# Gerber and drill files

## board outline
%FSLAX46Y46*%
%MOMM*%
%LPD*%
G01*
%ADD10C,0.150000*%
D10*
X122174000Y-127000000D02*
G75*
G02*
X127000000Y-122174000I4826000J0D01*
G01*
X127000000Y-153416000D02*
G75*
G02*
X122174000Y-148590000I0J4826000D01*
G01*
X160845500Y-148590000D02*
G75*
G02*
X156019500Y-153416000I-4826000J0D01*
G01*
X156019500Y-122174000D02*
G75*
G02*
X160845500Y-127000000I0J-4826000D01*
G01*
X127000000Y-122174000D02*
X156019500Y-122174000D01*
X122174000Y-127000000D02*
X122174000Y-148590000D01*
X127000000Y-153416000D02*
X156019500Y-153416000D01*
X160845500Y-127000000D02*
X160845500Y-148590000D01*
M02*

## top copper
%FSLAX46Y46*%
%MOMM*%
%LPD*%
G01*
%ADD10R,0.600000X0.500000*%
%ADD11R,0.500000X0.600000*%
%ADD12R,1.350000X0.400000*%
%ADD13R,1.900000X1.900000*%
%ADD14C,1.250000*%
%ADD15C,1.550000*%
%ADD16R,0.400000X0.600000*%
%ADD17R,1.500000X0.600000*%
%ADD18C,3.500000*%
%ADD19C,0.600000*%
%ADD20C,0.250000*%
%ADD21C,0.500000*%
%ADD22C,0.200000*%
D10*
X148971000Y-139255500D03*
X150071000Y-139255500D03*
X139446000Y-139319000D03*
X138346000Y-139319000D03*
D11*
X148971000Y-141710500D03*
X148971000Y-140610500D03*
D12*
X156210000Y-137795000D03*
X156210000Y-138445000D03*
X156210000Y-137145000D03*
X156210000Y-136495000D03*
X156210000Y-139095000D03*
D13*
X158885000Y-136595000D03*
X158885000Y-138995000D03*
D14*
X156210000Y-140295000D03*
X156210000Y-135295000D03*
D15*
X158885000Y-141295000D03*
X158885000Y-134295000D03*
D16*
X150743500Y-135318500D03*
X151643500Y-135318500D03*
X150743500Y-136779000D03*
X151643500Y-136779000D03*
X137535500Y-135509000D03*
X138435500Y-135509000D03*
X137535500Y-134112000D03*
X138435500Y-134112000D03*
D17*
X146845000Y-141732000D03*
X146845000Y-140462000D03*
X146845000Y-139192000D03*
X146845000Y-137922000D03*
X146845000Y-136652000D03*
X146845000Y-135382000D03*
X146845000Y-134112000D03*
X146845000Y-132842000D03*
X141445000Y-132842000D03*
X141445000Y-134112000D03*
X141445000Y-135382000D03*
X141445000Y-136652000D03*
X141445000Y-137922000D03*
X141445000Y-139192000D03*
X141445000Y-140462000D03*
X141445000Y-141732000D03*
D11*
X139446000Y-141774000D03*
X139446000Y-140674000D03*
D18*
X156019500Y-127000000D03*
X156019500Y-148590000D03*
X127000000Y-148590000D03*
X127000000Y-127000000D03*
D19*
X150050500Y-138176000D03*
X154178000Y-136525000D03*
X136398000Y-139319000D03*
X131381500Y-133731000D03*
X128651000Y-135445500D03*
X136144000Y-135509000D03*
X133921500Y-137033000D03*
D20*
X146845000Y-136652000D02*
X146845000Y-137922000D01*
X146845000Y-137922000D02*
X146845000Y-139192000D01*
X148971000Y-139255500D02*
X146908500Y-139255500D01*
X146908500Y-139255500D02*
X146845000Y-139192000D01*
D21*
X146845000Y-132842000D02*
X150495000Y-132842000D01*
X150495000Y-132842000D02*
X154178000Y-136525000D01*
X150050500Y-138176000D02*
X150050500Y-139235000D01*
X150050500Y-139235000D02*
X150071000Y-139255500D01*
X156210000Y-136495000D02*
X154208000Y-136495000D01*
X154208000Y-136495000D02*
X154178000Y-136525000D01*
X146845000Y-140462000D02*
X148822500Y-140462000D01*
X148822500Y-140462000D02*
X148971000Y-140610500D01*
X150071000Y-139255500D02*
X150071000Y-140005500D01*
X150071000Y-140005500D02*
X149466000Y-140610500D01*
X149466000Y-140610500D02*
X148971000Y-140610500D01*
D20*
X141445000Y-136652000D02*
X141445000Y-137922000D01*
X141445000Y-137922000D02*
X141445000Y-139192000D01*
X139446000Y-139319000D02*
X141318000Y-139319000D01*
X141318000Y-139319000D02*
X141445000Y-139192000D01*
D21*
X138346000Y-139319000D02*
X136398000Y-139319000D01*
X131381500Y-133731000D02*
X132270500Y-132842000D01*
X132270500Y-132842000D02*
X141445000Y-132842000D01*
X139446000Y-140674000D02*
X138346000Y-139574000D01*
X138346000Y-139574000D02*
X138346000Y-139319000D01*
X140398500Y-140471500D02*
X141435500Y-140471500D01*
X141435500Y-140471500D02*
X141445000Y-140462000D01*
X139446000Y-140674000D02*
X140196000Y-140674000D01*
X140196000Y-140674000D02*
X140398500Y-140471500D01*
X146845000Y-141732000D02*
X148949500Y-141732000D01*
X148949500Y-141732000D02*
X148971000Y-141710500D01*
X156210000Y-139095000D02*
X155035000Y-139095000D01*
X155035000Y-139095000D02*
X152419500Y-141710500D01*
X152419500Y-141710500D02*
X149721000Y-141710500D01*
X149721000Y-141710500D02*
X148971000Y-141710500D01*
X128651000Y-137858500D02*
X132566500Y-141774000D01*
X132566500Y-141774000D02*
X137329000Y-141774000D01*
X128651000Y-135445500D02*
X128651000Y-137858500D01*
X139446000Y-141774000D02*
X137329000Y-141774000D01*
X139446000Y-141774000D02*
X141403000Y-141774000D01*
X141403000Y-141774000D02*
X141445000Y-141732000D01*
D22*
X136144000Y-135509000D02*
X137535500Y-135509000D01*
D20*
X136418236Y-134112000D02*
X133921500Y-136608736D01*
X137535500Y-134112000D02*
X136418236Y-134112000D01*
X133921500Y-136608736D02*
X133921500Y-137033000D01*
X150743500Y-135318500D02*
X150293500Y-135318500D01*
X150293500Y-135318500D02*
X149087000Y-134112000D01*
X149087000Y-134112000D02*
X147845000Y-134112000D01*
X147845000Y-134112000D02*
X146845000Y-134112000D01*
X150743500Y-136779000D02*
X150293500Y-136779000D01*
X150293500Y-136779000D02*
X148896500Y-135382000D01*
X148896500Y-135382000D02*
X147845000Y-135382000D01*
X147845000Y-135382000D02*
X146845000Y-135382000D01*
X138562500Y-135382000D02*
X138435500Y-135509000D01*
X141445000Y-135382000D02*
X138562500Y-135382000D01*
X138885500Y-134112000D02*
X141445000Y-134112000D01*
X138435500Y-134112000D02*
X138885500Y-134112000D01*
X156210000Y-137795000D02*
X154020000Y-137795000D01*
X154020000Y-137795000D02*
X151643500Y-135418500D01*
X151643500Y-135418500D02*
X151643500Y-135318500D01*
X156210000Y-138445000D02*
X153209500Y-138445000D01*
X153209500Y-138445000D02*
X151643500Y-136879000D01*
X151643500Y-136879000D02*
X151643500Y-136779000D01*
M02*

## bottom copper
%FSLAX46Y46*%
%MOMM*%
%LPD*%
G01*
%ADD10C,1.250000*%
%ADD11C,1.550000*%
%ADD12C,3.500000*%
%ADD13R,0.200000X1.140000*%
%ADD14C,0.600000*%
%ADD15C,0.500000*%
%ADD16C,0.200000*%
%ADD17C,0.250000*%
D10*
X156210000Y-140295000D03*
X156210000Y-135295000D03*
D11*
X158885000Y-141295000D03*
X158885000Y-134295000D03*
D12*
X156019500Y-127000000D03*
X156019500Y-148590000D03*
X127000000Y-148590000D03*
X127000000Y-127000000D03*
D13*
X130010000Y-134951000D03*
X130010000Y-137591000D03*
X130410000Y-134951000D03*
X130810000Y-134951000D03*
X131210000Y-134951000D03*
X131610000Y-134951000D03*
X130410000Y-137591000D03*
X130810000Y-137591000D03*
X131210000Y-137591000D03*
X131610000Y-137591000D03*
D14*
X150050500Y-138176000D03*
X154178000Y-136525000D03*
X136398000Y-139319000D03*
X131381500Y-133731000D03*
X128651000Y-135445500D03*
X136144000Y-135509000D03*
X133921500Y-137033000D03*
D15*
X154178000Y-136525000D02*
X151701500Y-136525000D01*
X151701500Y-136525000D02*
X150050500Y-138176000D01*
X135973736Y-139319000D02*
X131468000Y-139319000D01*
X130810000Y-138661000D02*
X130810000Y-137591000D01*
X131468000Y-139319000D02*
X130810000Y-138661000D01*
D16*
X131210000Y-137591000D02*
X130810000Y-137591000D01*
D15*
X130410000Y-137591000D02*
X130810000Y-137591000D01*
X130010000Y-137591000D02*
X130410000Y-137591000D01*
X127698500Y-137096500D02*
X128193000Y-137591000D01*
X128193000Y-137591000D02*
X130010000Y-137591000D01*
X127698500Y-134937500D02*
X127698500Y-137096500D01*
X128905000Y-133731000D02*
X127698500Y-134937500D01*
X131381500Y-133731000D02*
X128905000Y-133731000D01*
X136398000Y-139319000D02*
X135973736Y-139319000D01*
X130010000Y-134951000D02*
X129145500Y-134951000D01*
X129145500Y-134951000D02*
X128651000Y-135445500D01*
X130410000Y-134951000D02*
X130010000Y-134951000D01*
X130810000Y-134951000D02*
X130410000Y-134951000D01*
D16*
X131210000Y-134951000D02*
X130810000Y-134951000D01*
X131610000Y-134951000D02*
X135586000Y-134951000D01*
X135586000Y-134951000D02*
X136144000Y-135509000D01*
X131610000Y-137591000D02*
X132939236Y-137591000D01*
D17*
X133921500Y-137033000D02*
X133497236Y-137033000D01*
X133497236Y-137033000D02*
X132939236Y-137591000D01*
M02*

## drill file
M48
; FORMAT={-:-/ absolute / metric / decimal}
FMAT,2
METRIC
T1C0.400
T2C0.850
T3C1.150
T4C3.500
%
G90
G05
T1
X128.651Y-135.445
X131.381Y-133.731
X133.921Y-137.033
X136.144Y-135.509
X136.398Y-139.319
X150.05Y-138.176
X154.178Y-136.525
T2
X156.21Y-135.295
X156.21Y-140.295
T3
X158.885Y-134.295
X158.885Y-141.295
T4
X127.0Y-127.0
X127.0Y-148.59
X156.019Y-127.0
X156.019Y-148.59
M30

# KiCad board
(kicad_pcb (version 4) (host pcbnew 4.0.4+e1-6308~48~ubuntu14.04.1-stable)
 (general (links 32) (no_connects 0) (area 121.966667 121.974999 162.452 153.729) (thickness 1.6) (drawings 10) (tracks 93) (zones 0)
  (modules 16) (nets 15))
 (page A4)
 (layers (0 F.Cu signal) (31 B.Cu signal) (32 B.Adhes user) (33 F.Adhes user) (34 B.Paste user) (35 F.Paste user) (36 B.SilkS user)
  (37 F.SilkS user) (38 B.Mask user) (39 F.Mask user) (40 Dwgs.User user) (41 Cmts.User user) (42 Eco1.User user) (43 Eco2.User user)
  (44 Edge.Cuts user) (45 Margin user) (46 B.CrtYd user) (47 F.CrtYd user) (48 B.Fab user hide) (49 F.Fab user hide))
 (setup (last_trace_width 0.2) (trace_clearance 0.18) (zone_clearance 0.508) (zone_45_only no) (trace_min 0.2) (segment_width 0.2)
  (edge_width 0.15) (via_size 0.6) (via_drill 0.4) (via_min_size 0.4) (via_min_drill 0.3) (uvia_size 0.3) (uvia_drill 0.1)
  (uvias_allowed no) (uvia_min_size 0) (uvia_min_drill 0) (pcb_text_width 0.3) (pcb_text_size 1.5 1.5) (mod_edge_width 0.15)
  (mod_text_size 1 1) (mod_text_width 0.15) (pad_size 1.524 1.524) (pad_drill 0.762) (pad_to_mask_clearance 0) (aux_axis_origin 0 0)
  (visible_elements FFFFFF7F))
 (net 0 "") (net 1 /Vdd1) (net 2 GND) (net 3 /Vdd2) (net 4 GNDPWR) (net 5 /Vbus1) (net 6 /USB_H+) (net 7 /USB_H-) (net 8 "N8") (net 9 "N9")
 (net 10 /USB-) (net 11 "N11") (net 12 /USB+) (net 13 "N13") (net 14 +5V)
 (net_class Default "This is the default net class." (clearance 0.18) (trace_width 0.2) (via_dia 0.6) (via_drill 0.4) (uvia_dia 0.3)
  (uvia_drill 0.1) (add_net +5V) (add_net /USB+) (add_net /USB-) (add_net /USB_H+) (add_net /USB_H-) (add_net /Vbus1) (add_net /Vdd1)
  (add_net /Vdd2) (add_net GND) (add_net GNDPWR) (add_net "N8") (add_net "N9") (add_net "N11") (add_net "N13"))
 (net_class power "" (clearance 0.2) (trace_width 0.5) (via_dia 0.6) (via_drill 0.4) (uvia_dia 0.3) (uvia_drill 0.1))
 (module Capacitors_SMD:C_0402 (layer F.Cu) (at 149.521 139.2555)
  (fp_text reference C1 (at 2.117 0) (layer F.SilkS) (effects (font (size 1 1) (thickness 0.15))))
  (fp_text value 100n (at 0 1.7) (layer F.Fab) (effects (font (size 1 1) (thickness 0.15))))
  (pad 1 smd rect (at -0.55 0) (size 0.6 0.5) (layers F.Cu F.Paste F.Mask) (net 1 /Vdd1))
  (pad 2 smd rect (at 0.55 0) (size 0.6 0.5) (layers F.Cu F.Paste F.Mask) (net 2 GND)))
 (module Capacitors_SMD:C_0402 (layer F.Cu) (at 138.896 139.319 180)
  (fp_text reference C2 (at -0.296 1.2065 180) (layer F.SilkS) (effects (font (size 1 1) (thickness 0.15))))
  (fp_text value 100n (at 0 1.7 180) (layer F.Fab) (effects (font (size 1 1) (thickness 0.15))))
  (pad 1 smd rect (at -0.55 0 180) (size 0.6 0.5) (layers F.Cu F.Paste F.Mask) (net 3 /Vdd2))
  (pad 2 smd rect (at 0.55 0 180) (size 0.6 0.5) (layers F.Cu F.Paste F.Mask) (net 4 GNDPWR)))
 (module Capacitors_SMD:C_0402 (layer F.Cu) (at 148.971 141.1605 90)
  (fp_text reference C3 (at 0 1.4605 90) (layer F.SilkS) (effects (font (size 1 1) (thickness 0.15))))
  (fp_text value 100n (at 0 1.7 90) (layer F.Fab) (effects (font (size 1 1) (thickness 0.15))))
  (pad 1 smd rect (at -0.55 0 90) (size 0.6 0.5) (layers F.Cu F.Paste F.Mask) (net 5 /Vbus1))
  (pad 2 smd rect (at 0.55 0 90) (size 0.6 0.5) (layers F.Cu F.Paste F.Mask) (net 2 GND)))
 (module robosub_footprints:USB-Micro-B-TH (layer F.Cu) (at 155.535 137.795 90)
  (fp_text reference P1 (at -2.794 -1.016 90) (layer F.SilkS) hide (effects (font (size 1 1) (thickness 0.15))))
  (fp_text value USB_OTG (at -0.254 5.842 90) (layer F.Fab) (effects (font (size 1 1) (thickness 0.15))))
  (pad 3 smd rect (at 0 0.675 90) (size 0.4 1.35) (layers F.Cu F.Paste F.Mask) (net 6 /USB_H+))
  (pad 2 smd rect (at -0.65 0.675 90) (size 0.4 1.35) (layers F.Cu F.Paste F.Mask) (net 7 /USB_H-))
  (pad 4 smd rect (at 0.65 0.675 90) (size 0.4 1.35) (layers F.Cu F.Paste F.Mask))
  (pad 5 smd rect (at 1.3 0.675 90) (size 0.4 1.35) (layers F.Cu F.Paste F.Mask) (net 2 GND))
  (pad 1 smd rect (at -1.3 0.675 90) (size 0.4 1.35) (layers F.Cu F.Paste F.Mask) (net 5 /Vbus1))
  (pad "" smd rect (at 1.2 3.35 90) (size 1.9 1.9) (layers F.Cu F.Paste F.Mask))
  (pad "" smd rect (at -1.2 3.35 90) (size 1.9 1.9) (layers F.Cu F.Paste F.Mask))
  (pad "" thru_hole circle (at -2.5 0.675 90) (size 1.25 1.25) (drill 0.85) (layers *.Cu *.Mask F.SilkS))
  (pad "" thru_hole circle (at 2.5 0.675 90) (size 1.25 1.25) (drill 0.85) (layers *.Cu *.Mask F.SilkS))
  (pad "" thru_hole circle (at -3.5 3.35 90) (size 1.55 1.55) (drill 1.15) (layers *.Cu *.Mask F.SilkS))
  (pad "" thru_hole circle (at 3.5 3.35 90) (size 1.55 1.55) (drill 1.15) (layers *.Cu *.Mask F.SilkS)))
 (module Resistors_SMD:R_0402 (layer F.Cu) (at 151.1935 135.3185)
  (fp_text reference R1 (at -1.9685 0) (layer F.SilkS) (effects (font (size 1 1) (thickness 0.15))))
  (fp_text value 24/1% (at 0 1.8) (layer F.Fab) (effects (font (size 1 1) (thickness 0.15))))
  (pad 1 smd rect (at -0.45 0) (size 0.4 0.6) (layers F.Cu F.Paste F.Mask) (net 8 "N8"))
  (pad 2 smd rect (at 0.45 0) (size 0.4 0.6) (layers F.Cu F.Paste F.Mask) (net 6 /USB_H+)))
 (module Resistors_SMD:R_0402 (layer F.Cu) (at 151.1935 136.779)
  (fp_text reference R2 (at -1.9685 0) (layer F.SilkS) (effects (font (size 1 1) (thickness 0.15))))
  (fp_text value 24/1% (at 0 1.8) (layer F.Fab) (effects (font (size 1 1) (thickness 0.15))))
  (pad 1 smd rect (at -0.45 0) (size 0.4 0.6) (layers F.Cu F.Paste F.Mask) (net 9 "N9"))
  (pad 2 smd rect (at 0.45 0) (size 0.4 0.6) (layers F.Cu F.Paste F.Mask) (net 7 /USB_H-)))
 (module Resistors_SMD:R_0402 (layer F.Cu) (at 137.9855 135.509)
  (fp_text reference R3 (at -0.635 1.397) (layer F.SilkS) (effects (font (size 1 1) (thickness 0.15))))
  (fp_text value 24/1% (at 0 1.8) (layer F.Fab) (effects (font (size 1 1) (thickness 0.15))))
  (pad 1 smd rect (at -0.45 0) (size 0.4 0.6) (layers F.Cu F.Paste F.Mask) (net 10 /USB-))
  (pad 2 smd rect (at 0.45 0) (size 0.4 0.6) (layers F.Cu F.Paste F.Mask) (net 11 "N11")))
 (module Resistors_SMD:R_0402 (layer F.Cu) (at 137.9855 134.112)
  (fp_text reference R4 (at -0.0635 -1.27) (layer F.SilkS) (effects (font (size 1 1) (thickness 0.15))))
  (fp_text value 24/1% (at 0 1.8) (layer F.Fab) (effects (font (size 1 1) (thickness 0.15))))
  (pad 1 smd rect (at -0.45 0) (size 0.4 0.6) (layers F.Cu F.Paste F.Mask) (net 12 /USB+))
  (pad 2 smd rect (at 0.45 0) (size 0.4 0.6) (layers F.Cu F.Paste F.Mask) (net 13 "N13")))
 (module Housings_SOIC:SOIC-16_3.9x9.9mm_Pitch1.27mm (layer F.Cu) (at 144.145 137.287 180)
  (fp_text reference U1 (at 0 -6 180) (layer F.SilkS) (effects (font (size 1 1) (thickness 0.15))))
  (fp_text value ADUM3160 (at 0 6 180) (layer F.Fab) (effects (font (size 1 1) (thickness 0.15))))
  (pad 1 smd rect (at -2.7 -4.445 180) (size 1.5 0.6) (layers F.Cu F.Paste F.Mask) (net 5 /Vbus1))
  (pad 2 smd rect (at -2.7 -3.175 180) (size 1.5 0.6) (layers F.Cu F.Paste F.Mask) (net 2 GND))
  (pad 3 smd rect (at -2.7 -1.905 180) (size 1.5 0.6) (layers F.Cu F.Paste F.Mask) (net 1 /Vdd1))
  (pad 4 smd rect (at -2.7 -0.635 180) (size 1.5 0.6) (layers F.Cu F.Paste F.Mask) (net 1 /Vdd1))
  (pad 5 smd rect (at -2.7 0.635 180) (size 1.5 0.6) (layers F.Cu F.Paste F.Mask) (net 1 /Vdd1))
  (pad 6 smd rect (at -2.7 1.905 180) (size 1.5 0.6) (layers F.Cu F.Paste F.Mask) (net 9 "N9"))
  (pad 7 smd rect (at -2.7 3.175 180) (size 1.5 0.6) (layers F.Cu F.Paste F.Mask) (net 8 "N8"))
  (pad 8 smd rect (at -2.7 4.445 180) (size 1.5 0.6) (layers F.Cu F.Paste F.Mask) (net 2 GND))
  (pad 9 smd rect (at 2.7 4.445 180) (size 1.5 0.6) (layers F.Cu F.Paste F.Mask) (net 4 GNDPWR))
  (pad 10 smd rect (at 2.7 3.175 180) (size 1.5 0.6) (layers F.Cu F.Paste F.Mask) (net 13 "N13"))
  (pad 11 smd rect (at 2.7 1.905 180) (size 1.5 0.6) (layers F.Cu F.Paste F.Mask) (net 11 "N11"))
  (pad 12 smd rect (at 2.7 0.635 180) (size 1.5 0.6) (layers F.Cu F.Paste F.Mask) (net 3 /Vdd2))
  (pad 13 smd rect (at 2.7 -0.635 180) (size 1.5 0.6) (layers F.Cu F.Paste F.Mask) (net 3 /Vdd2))
  (pad 14 smd rect (at 2.7 -1.905 180) (size 1.5 0.6) (layers F.Cu F.Paste F.Mask) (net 3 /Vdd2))
  (pad 15 smd rect (at 2.7 -3.175 180) (size 1.5 0.6) (layers F.Cu F.Paste F.Mask) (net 4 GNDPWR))
  (pad 16 smd rect (at 2.7 -4.445 180) (size 1.5 0.6) (layers F.Cu F.Paste F.Mask) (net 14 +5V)))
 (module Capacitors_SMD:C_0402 (layer F.Cu) (at 139.446 141.224 90)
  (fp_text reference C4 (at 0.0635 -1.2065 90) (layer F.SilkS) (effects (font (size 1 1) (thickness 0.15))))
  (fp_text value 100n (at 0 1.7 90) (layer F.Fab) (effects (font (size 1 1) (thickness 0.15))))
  (pad 1 smd rect (at -0.55 0 90) (size 0.6 0.5) (layers F.Cu F.Paste F.Mask) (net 14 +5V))
  (pad 2 smd rect (at 0.55 0 90) (size 0.6 0.5) (layers F.Cu F.Paste F.Mask) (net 4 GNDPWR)))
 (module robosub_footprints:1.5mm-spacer (layer F.Cu) (at 156.0195 127)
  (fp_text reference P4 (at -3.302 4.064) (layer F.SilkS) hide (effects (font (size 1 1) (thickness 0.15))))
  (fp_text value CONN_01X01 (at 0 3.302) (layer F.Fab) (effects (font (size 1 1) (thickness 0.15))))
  (pad "" thru_hole circle (at 0 0) (size 3.5 3.5) (drill 3.5) (layers *.Cu *.Mask F.SilkS)))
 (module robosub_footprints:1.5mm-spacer (layer F.Cu) (at 156.0195 148.59)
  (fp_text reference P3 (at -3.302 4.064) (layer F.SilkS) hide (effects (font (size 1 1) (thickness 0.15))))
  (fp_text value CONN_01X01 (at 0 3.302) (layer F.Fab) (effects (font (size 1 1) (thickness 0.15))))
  (pad "" thru_hole circle (at 0 0) (size 3.5 3.5) (drill 3.5) (layers *.Cu *.Mask F.SilkS)))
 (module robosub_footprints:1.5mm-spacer (layer F.Cu) (at 127 148.59)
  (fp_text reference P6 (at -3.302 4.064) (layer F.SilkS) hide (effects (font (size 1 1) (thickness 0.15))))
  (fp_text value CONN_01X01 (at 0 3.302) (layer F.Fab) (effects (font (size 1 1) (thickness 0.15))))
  (pad "" thru_hole circle (at 0 0) (size 3.5 3.5) (drill 3.5) (layers *.Cu *.Mask F.SilkS)))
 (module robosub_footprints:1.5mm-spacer (layer F.Cu) (at 127 127)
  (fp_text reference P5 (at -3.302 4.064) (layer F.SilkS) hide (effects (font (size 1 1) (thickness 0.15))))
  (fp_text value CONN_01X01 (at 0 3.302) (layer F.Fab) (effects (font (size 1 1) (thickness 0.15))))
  (pad "" thru_hole circle (at 0 0) (size 3.5 3.5) (drill 3.5) (layers *.Cu *.Mask F.SilkS)))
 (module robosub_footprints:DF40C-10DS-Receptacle (layer B.Cu) (at 130.81 136.271)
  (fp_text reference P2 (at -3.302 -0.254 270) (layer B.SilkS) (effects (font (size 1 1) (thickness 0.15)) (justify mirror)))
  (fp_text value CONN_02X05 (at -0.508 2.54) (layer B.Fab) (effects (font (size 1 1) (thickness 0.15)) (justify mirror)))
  (pad 1 smd rect (at -0.8 -1.32 270) (size 1.14 0.2) (layers B.Cu B.Paste B.Mask) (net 14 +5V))
  (pad 2 smd rect (at -0.8 1.32 270) (size 1.14 0.2) (layers B.Cu B.Paste B.Mask) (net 4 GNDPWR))
  (pad 3 smd rect (at -0.4 -1.32 270) (size 1.14 0.2) (layers B.Cu B.Paste B.Mask) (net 14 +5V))
  (pad 5 smd rect (at 0 -1.32 270) (size 1.14 0.2) (layers B.Cu B.Paste B.Mask) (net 14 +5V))
  (pad 7 smd rect (at 0.4 -1.32 270) (size 1.14 0.2) (layers B.Cu B.Paste B.Mask) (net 14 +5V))
  (pad 9 smd rect (at 0.8 -1.32 270) (size 1.14 0.2) (layers B.Cu B.Paste B.Mask) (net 10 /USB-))
  (pad 4 smd rect (at -0.4 1.32 270) (size 1.14 0.2) (layers B.Cu B.Paste B.Mask) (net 4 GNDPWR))
  (pad 6 smd rect (at 0 1.32 270) (size 1.14 0.2) (layers B.Cu B.Paste B.Mask) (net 4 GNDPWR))
  (pad 8 smd rect (at 0.4 1.32 270) (size 1.14 0.2) (layers B.Cu B.Paste B.Mask) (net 4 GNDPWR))
  (pad 10 smd rect (at 0.8 1.32 270) (size 1.14 0.2) (layers B.Cu B.Paste B.Mask) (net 12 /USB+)))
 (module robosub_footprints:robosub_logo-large (layer F.Cu) (at 141.6685 148.59)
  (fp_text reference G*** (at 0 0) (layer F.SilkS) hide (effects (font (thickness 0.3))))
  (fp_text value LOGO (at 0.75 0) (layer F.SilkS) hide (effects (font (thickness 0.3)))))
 (gr_arc (start 127 127) (end 122.174 127) (angle 90) (layer Edge.Cuts) (width 0.15))
 (gr_arc (start 127 148.59) (end 127 153.416) (angle 90) (layer Edge.Cuts) (width 0.15))
 (gr_arc (start 156.0195 148.59) (end 160.8455 148.59) (angle 90) (layer Edge.Cuts) (width 0.15))
 (gr_arc (start 156.0195 127) (end 156.0195 122.174) (angle 90) (layer Edge.Cuts) (width 0.15))
 (gr_line (start 127 122.174) (end 156.0195 122.174) (layer Edge.Cuts) (width 0.15))
 (gr_line (start 122.174 127) (end 122.174 148.59) (layer Edge.Cuts) (width 0.15))
 (gr_line (start 127 153.416) (end 156.0195 153.416) (layer Edge.Cuts) (width 0.15))
 (gr_line (start 160.8455 127) (end 160.8455 148.59) (layer Edge.Cuts) (width 0.15))
 (segment (start 146.845 136.652) (end 146.845 137.922) (width 0.25) (layer F.Cu) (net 1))
 (segment (start 146.845 137.922) (end 146.845 139.192) (width 0.25) (layer F.Cu) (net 1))
 (segment (start 148.971 139.2555) (end 146.9085 139.2555) (width 0.25) (layer F.Cu) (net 1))
 (segment (start 146.9085 139.2555) (end 146.845 139.192) (width 0.25) (layer F.Cu) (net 1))
 (segment (start 146.845 132.842) (end 150.495 132.842) (width 0.5) (layer F.Cu) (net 2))
 (segment (start 150.495 132.842) (end 154.178 136.525) (width 0.5) (layer F.Cu) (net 2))
 (segment (start 150.0505 138.176) (end 150.0505 139.235) (width 0.5) (layer F.Cu) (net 2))
 (segment (start 150.0505 139.235) (end 150.071 139.2555) (width 0.5) (layer F.Cu) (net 2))
 (segment (start 154.178 136.525) (end 151.7015 136.525) (width 0.5) (layer B.Cu) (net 2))
 (segment (start 151.7015 136.525) (end 150.0505 138.176) (width 0.5) (layer B.Cu) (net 2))
 (via (at 150.0505 138.176) (size 0.6) (drill 0.4) (layers F.Cu B.Cu) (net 2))
 (segment (start 156.21 136.495) (end 154.208 136.495) (width 0.5) (layer F.Cu) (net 2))
 (segment (start 154.208 136.495) (end 154.178 136.525) (width 0.5) (layer F.Cu) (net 2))
 (via (at 154.178 136.525) (size 0.6) (drill 0.4) (layers F.Cu B.Cu) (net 2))
 (segment (start 146.845 140.462) (end 148.8225 140.462) (width 0.5) (layer F.Cu) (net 2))
 (segment (start 148.8225 140.462) (end 148.971 140.6105) (width 0.5) (layer F.Cu) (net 2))
 (segment (start 150.071 139.2555) (end 150.071 140.0055) (width 0.5) (layer F.Cu) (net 2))
 (segment (start 150.071 140.0055) (end 149.466 140.6105) (width 0.5) (layer F.Cu) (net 2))
 (segment (start 149.466 140.6105) (end 148.971 140.6105) (width 0.5) (layer F.Cu) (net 2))
 (segment (start 141.445 136.652) (end 141.445 137.922) (width 0.25) (layer F.Cu) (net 3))
 (segment (start 141.445 137.922) (end 141.445 139.192) (width 0.25) (layer F.Cu) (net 3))
 (segment (start 139.446 139.319) (end 141.318 139.319) (width 0.25) (layer F.Cu) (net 3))
 (segment (start 141.318 139.319) (end 141.445 139.192) (width 0.25) (layer F.Cu) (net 3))
 (segment (start 135.973736 139.319) (end 131.468 139.319) (width 0.5) (layer B.Cu) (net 4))
 (segment (start 130.81 138.661) (end 130.81 137.591) (width 0.5) (layer B.Cu) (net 4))
 (segment (start 131.468 139.319) (end 130.81 138.661) (width 0.5) (layer B.Cu) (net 4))
 (segment (start 131.21 137.591) (end 130.81 137.591) (width 0.2) (layer B.Cu) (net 4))
 (segment (start 130.41 137.591) (end 130.81 137.591) (width 0.5) (layer B.Cu) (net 4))
 (segment (start 130.01 137.591) (end 130.41 137.591) (width 0.5) (layer B.Cu) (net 4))
 (segment (start 127.6985 137.0965) (end 128.193 137.591) (width 0.5) (layer B.Cu) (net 4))
 (segment (start 128.193 137.591) (end 130.01 137.591) (width 0.5) (layer B.Cu) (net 4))
 (segment (start 127.6985 134.9375) (end 127.6985 137.0965) (width 0.5) (layer B.Cu) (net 4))
 (segment (start 128.905 133.731) (end 127.6985 134.9375) (width 0.5) (layer B.Cu) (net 4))
 (segment (start 131.3815 133.731) (end 128.905 133.731) (width 0.5) (layer B.Cu) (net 4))
 (segment (start 136.398 139.319) (end 135.973736 139.319) (width 0.5) (layer B.Cu) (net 4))
 (via (at 136.398 139.319) (size 0.6) (drill 0.4) (layers F.Cu B.Cu) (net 4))
 (segment (start 138.346 139.319) (end 136.398 139.319) (width 0.5) (layer F.Cu) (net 4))
 (segment (start 131.3815 133.731) (end 132.2705 132.842) (width 0.5) (layer F.Cu) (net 4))
 (segment (start 132.2705 132.842) (end 141.445 132.842) (width 0.5) (layer F.Cu) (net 4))
 (via (at 131.3815 133.731) (size 0.6) (drill 0.4) (layers F.Cu B.Cu) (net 4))
 (segment (start 139.446 140.674) (end 138.346 139.574) (width 0.5) (layer F.Cu) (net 4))
 (segment (start 138.346 139.574) (end 138.346 139.319) (width 0.5) (layer F.Cu) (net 4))
 (segment (start 140.3985 140.4715) (end 141.4355 140.4715) (width 0.5) (layer F.Cu) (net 4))
 (segment (start 141.4355 140.4715) (end 141.445 140.462) (width 0.5) (layer F.Cu) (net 4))
 (segment (start 139.446 140.674) (end 140.196 140.674) (width 0.5) (layer F.Cu) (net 4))
 (segment (start 140.196 140.674) (end 140.3985 140.4715) (width 0.5) (layer F.Cu) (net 4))
 (segment (start 146.845 141.732) (end 148.9495 141.732) (width 0.5) (layer F.Cu) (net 5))
 (segment (start 148.9495 141.732) (end 148.971 141.7105) (width 0.5) (layer F.Cu) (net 5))
 (segment (start 156.21 139.095) (end 155.035 139.095) (width 0.5) (layer F.Cu) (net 5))
 (segment (start 155.035 139.095) (end 152.4195 141.7105) (width 0.5) (layer F.Cu) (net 5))
 (segment (start 152.4195 141.7105) (end 149.721 141.7105) (width 0.5) (layer F.Cu) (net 5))
 (segment (start 149.721 141.7105) (end 148.971 141.7105) (width 0.5) (layer F.Cu) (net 5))
 (segment (start 128.651 137.8585) (end 132.5665 141.774) (width 0.5) (layer F.Cu) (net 14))
 (segment (start 132.5665 141.774) (end 137.329 141.774) (width 0.5) (layer F.Cu) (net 14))
 (segment (start 128.651 135.4455) (end 128.651 137.8585) (width 0.5) (layer F.Cu) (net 14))
 (segment (start 130.01 134.951) (end 129.1455 134.951) (width 0.5) (layer B.Cu) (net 14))
 (segment (start 129.1455 134.951) (end 128.651 135.4455) (width 0.5) (layer B.Cu) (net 14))
 (via (at 128.651 135.4455) (size 0.6) (drill 0.4) (layers F.Cu B.Cu) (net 14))
 (segment (start 130.41 134.951) (end 130.01 134.951) (width 0.5) (layer B.Cu) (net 14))
 (segment (start 130.81 134.951) (end 130.41 134.951) (width 0.5) (layer B.Cu) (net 14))
 (segment (start 131.21 134.951) (end 130.81 134.951) (width 0.2) (layer B.Cu) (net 14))
 (segment (start 139.446 141.774) (end 137.329 141.774) (width 0.5) (layer F.Cu) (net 14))
 (segment (start 139.446 141.774) (end 141.403 141.774) (width 0.5) (layer F.Cu) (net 14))
 (segment (start 141.403 141.774) (end 141.445 141.732) (width 0.5) (layer F.Cu) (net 14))
 (segment (start 136.144 135.509) (end 137.5355 135.509) (width 0.2) (layer F.Cu) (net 10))
 (via (at 136.144 135.509) (size 0.6) (drill 0.4) (layers F.Cu B.Cu) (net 10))
 (segment (start 131.61 134.951) (end 135.586 134.951) (width 0.2) (layer B.Cu) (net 10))
 (segment (start 135.586 134.951) (end 136.144 135.509) (width 0.2) (layer B.Cu) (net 10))
 (segment (start 136.418236 134.112) (end 133.9215 136.608736) (width 0.25) (layer F.Cu) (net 12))
 (segment (start 137.5355 134.112) (end 136.418236 134.112) (width 0.25) (layer F.Cu) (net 12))
 (segment (start 133.9215 136.608736) (end 133.9215 137.033) (width 0.25) (layer F.Cu) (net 12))
 (segment (start 131.61 137.591) (end 132.939236 137.591) (width 0.2) (layer B.Cu) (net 12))
 (segment (start 133.9215 137.033) (end 133.497236 137.033) (width 0.25) (layer B.Cu) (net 12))
 (segment (start 133.497236 137.033) (end 132.939236 137.591) (width 0.25) (layer B.Cu) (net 12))
 (via (at 133.9215 137.033) (size 0.6) (drill 0.4) (layers F.Cu B.Cu) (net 12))
 (segment (start 150.7435 135.3185) (end 150.2935 135.3185) (width 0.25) (layer F.Cu) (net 8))
 (segment (start 150.2935 135.3185) (end 149.087 134.112) (width 0.25) (layer F.Cu) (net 8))
 (segment (start 149.087 134.112) (end 147.845 134.112) (width 0.25) (layer F.Cu) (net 8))
 (segment (start 147.845 134.112) (end 146.845 134.112) (width 0.25) (layer F.Cu) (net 8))
 (segment (start 150.7435 136.779) (end 150.2935 136.779) (width 0.25) (layer F.Cu) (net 9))
 (segment (start 150.2935 136.779) (end 148.8965 135.382) (width 0.25) (layer F.Cu) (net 9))
 (segment (start 148.8965 135.382) (end 147.845 135.382) (width 0.25) (layer F.Cu) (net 9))
 (segment (start 147.845 135.382) (end 146.845 135.382) (width 0.25) (layer F.Cu) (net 9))
 (segment (start 138.5625 135.382) (end 138.4355 135.509) (width 0.25) (layer F.Cu) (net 11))
 (segment (start 141.445 135.382) (end 138.5625 135.382) (width 0.25) (layer F.Cu) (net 11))
 (segment (start 138.8855 134.112) (end 141.445 134.112) (width 0.25) (layer F.Cu) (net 13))
 (segment (start 138.4355 134.112) (end 138.8855 134.112) (width 0.25) (layer F.Cu) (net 13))
 (segment (start 156.21 137.795) (end 154.02 137.795) (width 0.25) (layer F.Cu) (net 6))
 (segment (start 154.02 137.795) (end 151.6435 135.4185) (width 0.25) (layer F.Cu) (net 6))
 (segment (start 151.6435 135.4185) (end 151.6435 135.3185) (width 0.25) (layer F.Cu) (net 6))
 (segment (start 156.21 138.445) (end 153.2095 138.445) (width 0.25) (layer F.Cu) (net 7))
 (segment (start 153.2095 138.445) (end 151.6435 136.879) (width 0.25) (layer F.Cu) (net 7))
 (segment (start 151.6435 136.879) (end 151.6435 136.779) (width 0.25) (layer F.Cu) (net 7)))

